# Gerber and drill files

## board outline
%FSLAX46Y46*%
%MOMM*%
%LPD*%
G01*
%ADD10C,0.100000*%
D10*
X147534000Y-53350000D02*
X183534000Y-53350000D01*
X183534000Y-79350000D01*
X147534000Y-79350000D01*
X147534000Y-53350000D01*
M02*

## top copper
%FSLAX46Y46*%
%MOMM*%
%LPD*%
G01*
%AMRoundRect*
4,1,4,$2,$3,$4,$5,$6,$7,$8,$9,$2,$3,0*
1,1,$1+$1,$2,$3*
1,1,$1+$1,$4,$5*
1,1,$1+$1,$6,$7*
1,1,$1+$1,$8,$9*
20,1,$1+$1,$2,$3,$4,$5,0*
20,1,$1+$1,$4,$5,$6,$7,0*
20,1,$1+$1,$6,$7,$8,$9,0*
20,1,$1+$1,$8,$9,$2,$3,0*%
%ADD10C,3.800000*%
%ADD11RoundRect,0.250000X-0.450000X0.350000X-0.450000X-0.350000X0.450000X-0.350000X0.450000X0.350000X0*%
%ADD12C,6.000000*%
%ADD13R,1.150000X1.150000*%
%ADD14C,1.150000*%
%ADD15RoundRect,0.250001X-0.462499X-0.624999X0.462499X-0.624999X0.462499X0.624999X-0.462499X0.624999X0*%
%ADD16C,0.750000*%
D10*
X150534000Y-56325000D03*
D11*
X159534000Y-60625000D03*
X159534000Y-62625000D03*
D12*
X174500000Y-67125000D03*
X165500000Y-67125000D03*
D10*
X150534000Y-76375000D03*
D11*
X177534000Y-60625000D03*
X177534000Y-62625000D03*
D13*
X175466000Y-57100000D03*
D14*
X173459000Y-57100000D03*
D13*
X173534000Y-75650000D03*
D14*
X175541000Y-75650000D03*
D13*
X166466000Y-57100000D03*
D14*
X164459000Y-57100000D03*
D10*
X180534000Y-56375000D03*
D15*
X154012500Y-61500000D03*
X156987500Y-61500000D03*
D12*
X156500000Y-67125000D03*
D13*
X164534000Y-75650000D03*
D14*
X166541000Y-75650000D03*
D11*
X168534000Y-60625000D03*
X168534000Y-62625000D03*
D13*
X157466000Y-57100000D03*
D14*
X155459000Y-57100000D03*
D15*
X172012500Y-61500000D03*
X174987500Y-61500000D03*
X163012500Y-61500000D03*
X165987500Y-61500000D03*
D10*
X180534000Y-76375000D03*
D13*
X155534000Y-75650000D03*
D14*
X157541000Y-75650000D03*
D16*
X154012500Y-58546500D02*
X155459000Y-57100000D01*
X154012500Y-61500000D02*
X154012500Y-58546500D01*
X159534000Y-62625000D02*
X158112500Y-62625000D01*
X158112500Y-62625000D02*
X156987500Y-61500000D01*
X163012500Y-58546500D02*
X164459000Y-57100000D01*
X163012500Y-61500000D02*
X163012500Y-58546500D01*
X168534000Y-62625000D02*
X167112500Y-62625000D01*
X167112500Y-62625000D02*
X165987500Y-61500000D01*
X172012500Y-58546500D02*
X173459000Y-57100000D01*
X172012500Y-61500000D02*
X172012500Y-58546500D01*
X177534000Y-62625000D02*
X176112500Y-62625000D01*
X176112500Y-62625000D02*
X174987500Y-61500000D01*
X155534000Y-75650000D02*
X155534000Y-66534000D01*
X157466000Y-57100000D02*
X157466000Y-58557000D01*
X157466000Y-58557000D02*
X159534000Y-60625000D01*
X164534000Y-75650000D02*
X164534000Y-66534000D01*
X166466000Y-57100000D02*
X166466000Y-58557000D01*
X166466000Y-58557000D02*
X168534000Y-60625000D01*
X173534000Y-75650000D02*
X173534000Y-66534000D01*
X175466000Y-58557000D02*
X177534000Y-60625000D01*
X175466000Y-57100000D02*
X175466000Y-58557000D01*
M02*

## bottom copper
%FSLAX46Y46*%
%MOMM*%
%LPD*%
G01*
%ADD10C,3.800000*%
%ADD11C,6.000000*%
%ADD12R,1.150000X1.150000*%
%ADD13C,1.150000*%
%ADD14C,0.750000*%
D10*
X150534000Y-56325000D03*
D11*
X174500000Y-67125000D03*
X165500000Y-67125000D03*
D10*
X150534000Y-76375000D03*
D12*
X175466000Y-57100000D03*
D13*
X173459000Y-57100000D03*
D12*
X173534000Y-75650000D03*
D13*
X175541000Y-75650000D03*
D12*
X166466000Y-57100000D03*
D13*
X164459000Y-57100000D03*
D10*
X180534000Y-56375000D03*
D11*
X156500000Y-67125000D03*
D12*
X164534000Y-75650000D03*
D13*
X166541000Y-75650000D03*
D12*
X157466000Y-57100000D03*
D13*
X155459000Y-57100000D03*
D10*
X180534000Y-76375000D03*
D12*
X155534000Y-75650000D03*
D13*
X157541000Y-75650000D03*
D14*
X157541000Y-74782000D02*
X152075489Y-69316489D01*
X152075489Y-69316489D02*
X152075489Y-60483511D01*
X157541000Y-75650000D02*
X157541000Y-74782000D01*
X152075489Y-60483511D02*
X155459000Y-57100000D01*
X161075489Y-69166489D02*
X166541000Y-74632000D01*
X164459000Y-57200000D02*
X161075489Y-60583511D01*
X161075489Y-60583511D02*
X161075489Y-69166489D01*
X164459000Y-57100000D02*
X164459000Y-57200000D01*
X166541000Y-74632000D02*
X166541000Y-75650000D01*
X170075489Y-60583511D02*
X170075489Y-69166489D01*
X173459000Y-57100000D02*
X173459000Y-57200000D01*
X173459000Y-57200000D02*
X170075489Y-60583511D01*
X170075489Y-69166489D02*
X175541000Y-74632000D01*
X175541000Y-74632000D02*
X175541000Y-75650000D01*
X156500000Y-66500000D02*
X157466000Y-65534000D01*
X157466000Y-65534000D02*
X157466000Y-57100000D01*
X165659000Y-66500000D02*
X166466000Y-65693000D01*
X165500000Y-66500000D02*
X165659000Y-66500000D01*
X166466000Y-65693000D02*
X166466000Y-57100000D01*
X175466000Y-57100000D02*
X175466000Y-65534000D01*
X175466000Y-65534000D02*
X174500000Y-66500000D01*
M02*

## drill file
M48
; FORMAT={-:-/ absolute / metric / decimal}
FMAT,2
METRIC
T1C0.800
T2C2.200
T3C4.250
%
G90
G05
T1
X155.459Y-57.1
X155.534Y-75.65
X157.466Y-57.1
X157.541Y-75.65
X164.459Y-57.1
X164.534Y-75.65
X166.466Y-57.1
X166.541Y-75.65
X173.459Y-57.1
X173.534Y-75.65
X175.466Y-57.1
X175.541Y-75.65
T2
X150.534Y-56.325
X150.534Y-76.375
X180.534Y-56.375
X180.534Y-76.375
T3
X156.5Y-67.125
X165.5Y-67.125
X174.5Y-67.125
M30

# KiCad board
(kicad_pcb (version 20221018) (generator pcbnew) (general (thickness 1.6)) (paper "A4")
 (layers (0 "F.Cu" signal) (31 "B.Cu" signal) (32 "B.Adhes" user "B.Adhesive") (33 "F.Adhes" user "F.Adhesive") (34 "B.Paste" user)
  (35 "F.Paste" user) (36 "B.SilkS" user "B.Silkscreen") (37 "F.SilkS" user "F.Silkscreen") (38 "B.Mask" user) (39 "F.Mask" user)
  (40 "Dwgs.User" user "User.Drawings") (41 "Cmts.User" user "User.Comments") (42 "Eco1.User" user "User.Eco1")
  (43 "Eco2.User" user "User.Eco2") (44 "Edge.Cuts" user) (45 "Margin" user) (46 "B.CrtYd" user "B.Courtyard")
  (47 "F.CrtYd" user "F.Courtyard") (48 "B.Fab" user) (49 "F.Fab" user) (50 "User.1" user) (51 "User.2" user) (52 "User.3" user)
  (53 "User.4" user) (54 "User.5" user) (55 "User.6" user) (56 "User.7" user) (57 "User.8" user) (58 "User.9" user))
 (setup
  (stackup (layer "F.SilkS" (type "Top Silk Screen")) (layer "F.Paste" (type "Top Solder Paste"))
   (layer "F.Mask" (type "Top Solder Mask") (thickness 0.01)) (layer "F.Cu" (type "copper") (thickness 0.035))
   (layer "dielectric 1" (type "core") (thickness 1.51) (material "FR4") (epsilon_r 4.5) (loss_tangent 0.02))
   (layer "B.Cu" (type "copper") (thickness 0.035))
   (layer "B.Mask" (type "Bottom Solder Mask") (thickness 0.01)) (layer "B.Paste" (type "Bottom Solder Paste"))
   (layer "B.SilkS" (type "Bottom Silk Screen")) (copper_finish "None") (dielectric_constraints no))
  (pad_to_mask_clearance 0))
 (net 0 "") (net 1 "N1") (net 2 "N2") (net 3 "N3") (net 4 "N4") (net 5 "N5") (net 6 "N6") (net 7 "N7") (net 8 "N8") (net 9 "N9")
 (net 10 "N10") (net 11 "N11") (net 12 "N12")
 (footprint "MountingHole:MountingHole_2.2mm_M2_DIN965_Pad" (layer "F.Cu") (at 150.534 56.375)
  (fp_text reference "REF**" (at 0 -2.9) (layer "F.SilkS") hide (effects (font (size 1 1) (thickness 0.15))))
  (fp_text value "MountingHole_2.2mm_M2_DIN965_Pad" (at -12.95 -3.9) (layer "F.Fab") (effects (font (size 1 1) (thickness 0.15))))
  (pad "1" thru_hole circle (at 0 -0.05) (size 3.8 3.8) (drill 2.2) (layers "*.Cu" "*.Mask")))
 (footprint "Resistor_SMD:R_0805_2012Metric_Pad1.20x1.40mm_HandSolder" (layer "F.Cu") (at 159.534 61.625 -90)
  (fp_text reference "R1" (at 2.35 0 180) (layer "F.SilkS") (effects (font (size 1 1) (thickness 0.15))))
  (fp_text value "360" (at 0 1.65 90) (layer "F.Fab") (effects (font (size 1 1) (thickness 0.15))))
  (pad "1" smd roundrect (at -1 0 270) (size 1.2 1.4) (layers "F.Cu" "F.Paste" "F.Mask") (roundrect_rratio 0.2083333333) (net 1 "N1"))
  (pad "2" smd roundrect (at 1 0 270) (size 1.2 1.4) (layers "F.Cu" "F.Paste" "F.Mask") (roundrect_rratio 0.2083333333) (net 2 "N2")))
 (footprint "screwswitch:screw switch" (layer "F.Cu") (at 174.5 67.125)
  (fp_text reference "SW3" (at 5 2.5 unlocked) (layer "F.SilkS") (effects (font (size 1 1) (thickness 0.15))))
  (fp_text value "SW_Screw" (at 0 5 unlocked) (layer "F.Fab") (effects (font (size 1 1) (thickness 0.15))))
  (pad "" np_thru_hole circle (at 0 0) (size 6 6) (drill 4.25) (layers "F&B.Cu" "*.Mask")))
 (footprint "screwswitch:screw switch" (layer "F.Cu") (at 165.5 67.125)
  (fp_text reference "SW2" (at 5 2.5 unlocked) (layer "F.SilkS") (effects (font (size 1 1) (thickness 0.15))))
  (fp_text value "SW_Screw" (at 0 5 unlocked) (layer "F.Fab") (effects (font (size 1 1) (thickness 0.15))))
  (pad "" np_thru_hole circle (at 0 0) (size 6 6) (drill 4.25) (layers "F&B.Cu" "*.Mask")))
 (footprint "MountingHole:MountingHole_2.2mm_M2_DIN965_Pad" (layer "F.Cu") (at 150.534 76.375)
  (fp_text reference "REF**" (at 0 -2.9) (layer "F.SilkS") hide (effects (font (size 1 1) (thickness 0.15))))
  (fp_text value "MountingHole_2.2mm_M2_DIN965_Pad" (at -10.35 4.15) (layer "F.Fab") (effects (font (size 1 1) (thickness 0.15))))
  (pad "1" thru_hole circle (at 0 0) (size 3.8 3.8) (drill 2.2) (layers "*.Cu" "*.Mask")))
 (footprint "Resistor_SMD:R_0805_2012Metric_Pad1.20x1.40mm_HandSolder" (layer "F.Cu") (at 177.534 61.625 -90)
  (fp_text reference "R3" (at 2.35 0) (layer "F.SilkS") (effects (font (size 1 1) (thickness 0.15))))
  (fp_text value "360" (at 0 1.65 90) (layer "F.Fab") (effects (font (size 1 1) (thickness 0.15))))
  (pad "1" smd roundrect (at -1 0 270) (size 1.2 1.4) (layers "F.Cu" "F.Paste" "F.Mask") (roundrect_rratio 0.2083333333) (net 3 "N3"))
  (pad "2" smd roundrect (at 1 0 270) (size 1.2 1.4) (layers "F.Cu" "F.Paste" "F.Mask") (roundrect_rratio 0.2083333333) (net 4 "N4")))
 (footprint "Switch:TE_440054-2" (layer "F.Cu") (at 175.466 57.1 180)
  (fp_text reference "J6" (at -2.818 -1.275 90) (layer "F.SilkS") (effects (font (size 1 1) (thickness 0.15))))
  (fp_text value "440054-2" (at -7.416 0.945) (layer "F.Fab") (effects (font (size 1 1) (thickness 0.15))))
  (pad "1" thru_hole rect (at 0 0 180) (size 1.15 1.15) (drill 0.8) (layers "*.Cu" "*.Mask") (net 3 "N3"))
  (pad "2" thru_hole circle (at 2.007 0 180) (size 1.15 1.15) (drill 0.8) (layers "*.Cu" "*.Mask") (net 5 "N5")))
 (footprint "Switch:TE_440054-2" (layer "F.Cu") (at 173.534 75.65)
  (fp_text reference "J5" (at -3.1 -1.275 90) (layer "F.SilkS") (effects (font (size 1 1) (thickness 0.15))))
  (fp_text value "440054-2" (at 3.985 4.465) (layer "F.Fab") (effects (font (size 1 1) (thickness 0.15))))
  (pad "1" thru_hole rect (at 0 0) (size 1.15 1.15) (drill 0.8) (layers "*.Cu" "*.Mask") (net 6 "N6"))
  (pad "2" thru_hole circle (at 2.007 0) (size 1.15 1.15) (drill 0.8) (layers "*.Cu" "*.Mask") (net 5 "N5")))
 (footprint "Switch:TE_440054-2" (layer "F.Cu") (at 166.466 57.1 180)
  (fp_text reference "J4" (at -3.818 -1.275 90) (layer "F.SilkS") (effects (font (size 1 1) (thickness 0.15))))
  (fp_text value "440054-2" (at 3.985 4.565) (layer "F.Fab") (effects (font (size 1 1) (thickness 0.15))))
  (pad "1" thru_hole rect (at 0 0 180) (size 1.15 1.15) (drill 0.8) (layers "*.Cu" "*.Mask") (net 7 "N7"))
  (pad "2" thru_hole circle (at 2.007 0 180) (size 1.15 1.15) (drill 0.8) (layers "*.Cu" "*.Mask") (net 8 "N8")))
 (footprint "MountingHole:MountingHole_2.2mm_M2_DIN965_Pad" (layer "F.Cu") (at 180.534 56.375)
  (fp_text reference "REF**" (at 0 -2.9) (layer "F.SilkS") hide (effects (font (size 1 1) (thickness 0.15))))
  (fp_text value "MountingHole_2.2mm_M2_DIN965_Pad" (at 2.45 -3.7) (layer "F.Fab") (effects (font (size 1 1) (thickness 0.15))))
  (pad "1" thru_hole circle (at 0 0) (size 3.8 3.8) (drill 2.2) (layers "*.Cu" "*.Mask")))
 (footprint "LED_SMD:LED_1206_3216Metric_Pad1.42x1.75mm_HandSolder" (layer "F.Cu") (at 155.5 61.5)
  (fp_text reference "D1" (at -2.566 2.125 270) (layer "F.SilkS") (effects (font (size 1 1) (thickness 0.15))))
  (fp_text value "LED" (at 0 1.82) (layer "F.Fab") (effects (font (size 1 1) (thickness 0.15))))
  (pad "1" smd roundrect (at -1.4875 0) (size 1.425 1.75) (layers "F.Cu" "F.Paste" "F.Mask") (roundrect_rratio 0.1754392982) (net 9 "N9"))
  (pad "2" smd roundrect (at 1.4875 0) (size 1.425 1.75) (layers "F.Cu" "F.Paste" "F.Mask") (roundrect_rratio 0.1754392982) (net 2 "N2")))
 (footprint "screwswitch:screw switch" (layer "F.Cu") (at 156.5 67.125)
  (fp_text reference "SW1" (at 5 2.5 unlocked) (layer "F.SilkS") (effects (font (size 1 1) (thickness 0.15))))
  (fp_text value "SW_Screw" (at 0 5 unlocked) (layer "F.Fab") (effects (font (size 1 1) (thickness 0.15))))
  (pad "" np_thru_hole circle (at 0 0) (size 6 6) (drill 4.25) (layers "F&B.Cu" "*.Mask")))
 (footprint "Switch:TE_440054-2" (layer "F.Cu") (at 164.534 75.65)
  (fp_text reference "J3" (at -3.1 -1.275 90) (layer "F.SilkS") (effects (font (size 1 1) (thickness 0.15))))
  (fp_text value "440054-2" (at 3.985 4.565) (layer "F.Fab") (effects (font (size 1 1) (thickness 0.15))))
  (pad "1" thru_hole rect (at 0 0) (size 1.15 1.15) (drill 0.8) (layers "*.Cu" "*.Mask") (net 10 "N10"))
  (pad "2" thru_hole circle (at 2.007 0) (size 1.15 1.15) (drill 0.8) (layers "*.Cu" "*.Mask") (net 8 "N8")))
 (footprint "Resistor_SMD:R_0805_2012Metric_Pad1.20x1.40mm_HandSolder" (layer "F.Cu") (at 168.534 61.625 -90)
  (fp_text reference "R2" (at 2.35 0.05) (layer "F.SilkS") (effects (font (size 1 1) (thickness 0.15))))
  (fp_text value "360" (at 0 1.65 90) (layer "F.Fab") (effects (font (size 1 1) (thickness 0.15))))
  (pad "1" smd roundrect (at -1 0 270) (size 1.2 1.4) (layers "F.Cu" "F.Paste" "F.Mask") (roundrect_rratio 0.2083333333) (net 7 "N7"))
  (pad "2" smd roundrect (at 1 0 270) (size 1.2 1.4) (layers "F.Cu" "F.Paste" "F.Mask") (roundrect_rratio 0.2083333333) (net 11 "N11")))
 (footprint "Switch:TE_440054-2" (layer "F.Cu") (at 157.466 57.1 180)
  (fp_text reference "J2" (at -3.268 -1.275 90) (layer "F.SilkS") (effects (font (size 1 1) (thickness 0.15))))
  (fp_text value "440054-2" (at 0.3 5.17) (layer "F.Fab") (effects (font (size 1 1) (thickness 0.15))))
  (pad "1" thru_hole rect (at 0 0 180) (size 1.15 1.15) (drill 0.8) (layers "*.Cu" "*.Mask") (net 1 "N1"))
  (pad "2" thru_hole circle (at 2.007 0 180) (size 1.15 1.15) (drill 0.8) (layers "*.Cu" "*.Mask") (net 9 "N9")))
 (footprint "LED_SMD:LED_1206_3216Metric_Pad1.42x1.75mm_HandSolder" (layer "F.Cu") (at 173.5 61.5)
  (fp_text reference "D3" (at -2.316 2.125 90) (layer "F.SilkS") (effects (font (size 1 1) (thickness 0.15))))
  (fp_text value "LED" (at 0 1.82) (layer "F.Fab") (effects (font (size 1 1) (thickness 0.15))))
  (pad "1" smd roundrect (at -1.4875 0) (size 1.425 1.75) (layers "F.Cu" "F.Paste" "F.Mask") (roundrect_rratio 0.1754392982) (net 5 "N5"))
  (pad "2" smd roundrect (at 1.4875 0) (size 1.425 1.75) (layers "F.Cu" "F.Paste" "F.Mask") (roundrect_rratio 0.1754392982) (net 4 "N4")))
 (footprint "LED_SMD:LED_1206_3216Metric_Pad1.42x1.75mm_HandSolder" (layer "F.Cu") (at 164.5 61.5)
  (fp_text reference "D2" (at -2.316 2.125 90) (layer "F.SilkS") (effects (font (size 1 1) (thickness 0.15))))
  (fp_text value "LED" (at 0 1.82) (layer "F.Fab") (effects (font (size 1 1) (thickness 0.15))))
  (pad "1" smd roundrect (at -1.4875 0) (size 1.425 1.75) (layers "F.Cu" "F.Paste" "F.Mask") (roundrect_rratio 0.1754392982) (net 8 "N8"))
  (pad "2" smd roundrect (at 1.4875 0) (size 1.425 1.75) (layers "F.Cu" "F.Paste" "F.Mask") (roundrect_rratio 0.1754392982) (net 11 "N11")))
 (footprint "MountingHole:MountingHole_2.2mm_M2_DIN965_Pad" (layer "F.Cu") (at 180.534 76.375)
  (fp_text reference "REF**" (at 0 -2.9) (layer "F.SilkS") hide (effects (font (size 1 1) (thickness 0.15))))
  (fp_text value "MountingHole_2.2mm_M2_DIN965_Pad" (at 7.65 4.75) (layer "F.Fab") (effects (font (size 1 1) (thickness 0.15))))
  (pad "1" thru_hole circle (at 0 0) (size 3.8 3.8) (drill 2.2) (layers "*.Cu" "*.Mask")))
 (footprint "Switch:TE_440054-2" (layer "F.Cu") (at 155.534 75.65)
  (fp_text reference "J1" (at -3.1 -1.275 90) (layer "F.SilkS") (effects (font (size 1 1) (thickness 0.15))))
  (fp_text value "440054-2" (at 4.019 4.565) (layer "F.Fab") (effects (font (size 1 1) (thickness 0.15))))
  (pad "1" thru_hole rect (at 0 0) (size 1.15 1.15) (drill 0.8) (layers "*.Cu" "*.Mask") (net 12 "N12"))
  (pad "2" thru_hole circle (at 2.007 0) (size 1.15 1.15) (drill 0.8) (layers "*.Cu" "*.Mask") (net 9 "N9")))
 (gr_rect (start 147.534 53.35) (end 183.534 79.35) (stroke (width 0.1) (type solid)) (fill none) (layer "Edge.Cuts"))
 (segment (start 154.0125 58.5465) (end 155.459 57.1) (width 0.75) (layer "F.Cu") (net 9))
 (segment (start 154.0125 61.5) (end 154.0125 58.5465) (width 0.75) (layer "F.Cu") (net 9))
 (segment (start 157.541 74.782) (end 152.075489 69.316489) (width 0.75) (layer "B.Cu") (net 9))
 (segment (start 152.075489 69.316489) (end 152.075489 60.483511) (width 0.75) (layer "B.Cu") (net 9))
 (segment (start 157.541 75.65) (end 157.541 74.782) (width 0.75) (layer "B.Cu") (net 9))
 (segment (start 152.075489 60.483511) (end 155.459 57.1) (width 0.75) (layer "B.Cu") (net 9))
 (segment (start 159.534 62.625) (end 158.1125 62.625) (width 0.75) (layer "F.Cu") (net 2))
 (segment (start 158.1125 62.625) (end 156.9875 61.5) (width 0.75) (layer "F.Cu") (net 2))
 (segment (start 163.0125 58.5465) (end 164.459 57.1) (width 0.75) (layer "F.Cu") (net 8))
 (segment (start 163.0125 61.5) (end 163.0125 58.5465) (width 0.75) (layer "F.Cu") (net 8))
 (segment (start 161.075489 69.166489) (end 166.541 74.632) (width 0.75) (layer "B.Cu") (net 8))
 (segment (start 164.459 57.2) (end 161.075489 60.583511) (width 0.75) (layer "B.Cu") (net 8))
 (segment (start 161.075489 60.583511) (end 161.075489 69.166489) (width 0.75) (layer "B.Cu") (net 8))
 (segment (start 164.459 57.1) (end 164.459 57.2) (width 0.75) (layer "B.Cu") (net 8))
 (segment (start 166.541 74.632) (end 166.541 75.65) (width 0.75) (layer "B.Cu") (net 8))
 (segment (start 168.534 62.625) (end 167.1125 62.625) (width 0.75) (layer "F.Cu") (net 11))
 (segment (start 167.1125 62.625) (end 165.9875 61.5) (width 0.75) (layer "F.Cu") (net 11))
 (segment (start 172.0125 58.5465) (end 173.459 57.1) (width 0.75) (layer "F.Cu") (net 5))
 (segment (start 172.0125 61.5) (end 172.0125 58.5465) (width 0.75) (layer "F.Cu") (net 5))
 (segment (start 170.075489 60.583511) (end 170.075489 69.166489) (width 0.75) (layer "B.Cu") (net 5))
 (segment (start 173.459 57.1) (end 173.459 57.2) (width 0.75) (layer "B.Cu") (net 5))
 (segment (start 173.459 57.2) (end 170.075489 60.583511) (width 0.75) (layer "B.Cu") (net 5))
 (segment (start 170.075489 69.166489) (end 175.541 74.632) (width 0.75) (layer "B.Cu") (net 5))
 (segment (start 175.541 74.632) (end 175.541 75.65) (width 0.75) (layer "B.Cu") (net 5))
 (segment (start 177.534 62.625) (end 176.1125 62.625) (width 0.75) (layer "F.Cu") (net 4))
 (segment (start 176.1125 62.625) (end 174.9875 61.5) (width 0.75) (layer "F.Cu") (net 4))
 (segment (start 155.534 75.65) (end 155.534 66.534) (width 0.75) (layer "F.Cu") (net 12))
 (segment (start 157.466 57.1) (end 157.466 58.557) (width 0.75) (layer "F.Cu") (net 1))
 (segment (start 157.466 58.557) (end 159.534 60.625) (width 0.75) (layer "F.Cu") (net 1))
 (segment (start 156.5 66.5) (end 157.466 65.534) (width 0.75) (layer "B.Cu") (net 1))
 (segment (start 157.466 65.534) (end 157.466 57.1) (width 0.75) (layer "B.Cu") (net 1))
 (segment (start 164.534 75.65) (end 164.534 66.534) (width 0.75) (layer "F.Cu") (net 10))
 (segment (start 166.466 57.1) (end 166.466 58.557) (width 0.75) (layer "F.Cu") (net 7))
 (segment (start 166.466 58.557) (end 168.534 60.625) (width 0.75) (layer "F.Cu") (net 7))
 (segment (start 165.659 66.5) (end 166.466 65.693) (width 0.75) (layer "B.Cu") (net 7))
 (segment (start 165.5 66.5) (end 165.659 66.5) (width 0.75) (layer "B.Cu") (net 7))
 (segment (start 166.466 65.693) (end 166.466 57.1) (width 0.75) (layer "B.Cu") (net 7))
 (segment (start 173.534 75.65) (end 173.534 66.534) (width 0.75) (layer "F.Cu") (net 6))
 (segment (start 175.466 58.557) (end 177.534 60.625) (width 0.75) (layer "F.Cu") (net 3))
 (segment (start 175.466 57.1) (end 175.466 58.557) (width 0.75) (layer "F.Cu") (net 3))
 (segment (start 175.466 57.1) (end 175.466 65.534) (width 0.75) (layer "B.Cu") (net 3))
 (segment (start 175.466 65.534) (end 174.5 66.5) (width 0.75) (layer "B.Cu") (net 3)))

